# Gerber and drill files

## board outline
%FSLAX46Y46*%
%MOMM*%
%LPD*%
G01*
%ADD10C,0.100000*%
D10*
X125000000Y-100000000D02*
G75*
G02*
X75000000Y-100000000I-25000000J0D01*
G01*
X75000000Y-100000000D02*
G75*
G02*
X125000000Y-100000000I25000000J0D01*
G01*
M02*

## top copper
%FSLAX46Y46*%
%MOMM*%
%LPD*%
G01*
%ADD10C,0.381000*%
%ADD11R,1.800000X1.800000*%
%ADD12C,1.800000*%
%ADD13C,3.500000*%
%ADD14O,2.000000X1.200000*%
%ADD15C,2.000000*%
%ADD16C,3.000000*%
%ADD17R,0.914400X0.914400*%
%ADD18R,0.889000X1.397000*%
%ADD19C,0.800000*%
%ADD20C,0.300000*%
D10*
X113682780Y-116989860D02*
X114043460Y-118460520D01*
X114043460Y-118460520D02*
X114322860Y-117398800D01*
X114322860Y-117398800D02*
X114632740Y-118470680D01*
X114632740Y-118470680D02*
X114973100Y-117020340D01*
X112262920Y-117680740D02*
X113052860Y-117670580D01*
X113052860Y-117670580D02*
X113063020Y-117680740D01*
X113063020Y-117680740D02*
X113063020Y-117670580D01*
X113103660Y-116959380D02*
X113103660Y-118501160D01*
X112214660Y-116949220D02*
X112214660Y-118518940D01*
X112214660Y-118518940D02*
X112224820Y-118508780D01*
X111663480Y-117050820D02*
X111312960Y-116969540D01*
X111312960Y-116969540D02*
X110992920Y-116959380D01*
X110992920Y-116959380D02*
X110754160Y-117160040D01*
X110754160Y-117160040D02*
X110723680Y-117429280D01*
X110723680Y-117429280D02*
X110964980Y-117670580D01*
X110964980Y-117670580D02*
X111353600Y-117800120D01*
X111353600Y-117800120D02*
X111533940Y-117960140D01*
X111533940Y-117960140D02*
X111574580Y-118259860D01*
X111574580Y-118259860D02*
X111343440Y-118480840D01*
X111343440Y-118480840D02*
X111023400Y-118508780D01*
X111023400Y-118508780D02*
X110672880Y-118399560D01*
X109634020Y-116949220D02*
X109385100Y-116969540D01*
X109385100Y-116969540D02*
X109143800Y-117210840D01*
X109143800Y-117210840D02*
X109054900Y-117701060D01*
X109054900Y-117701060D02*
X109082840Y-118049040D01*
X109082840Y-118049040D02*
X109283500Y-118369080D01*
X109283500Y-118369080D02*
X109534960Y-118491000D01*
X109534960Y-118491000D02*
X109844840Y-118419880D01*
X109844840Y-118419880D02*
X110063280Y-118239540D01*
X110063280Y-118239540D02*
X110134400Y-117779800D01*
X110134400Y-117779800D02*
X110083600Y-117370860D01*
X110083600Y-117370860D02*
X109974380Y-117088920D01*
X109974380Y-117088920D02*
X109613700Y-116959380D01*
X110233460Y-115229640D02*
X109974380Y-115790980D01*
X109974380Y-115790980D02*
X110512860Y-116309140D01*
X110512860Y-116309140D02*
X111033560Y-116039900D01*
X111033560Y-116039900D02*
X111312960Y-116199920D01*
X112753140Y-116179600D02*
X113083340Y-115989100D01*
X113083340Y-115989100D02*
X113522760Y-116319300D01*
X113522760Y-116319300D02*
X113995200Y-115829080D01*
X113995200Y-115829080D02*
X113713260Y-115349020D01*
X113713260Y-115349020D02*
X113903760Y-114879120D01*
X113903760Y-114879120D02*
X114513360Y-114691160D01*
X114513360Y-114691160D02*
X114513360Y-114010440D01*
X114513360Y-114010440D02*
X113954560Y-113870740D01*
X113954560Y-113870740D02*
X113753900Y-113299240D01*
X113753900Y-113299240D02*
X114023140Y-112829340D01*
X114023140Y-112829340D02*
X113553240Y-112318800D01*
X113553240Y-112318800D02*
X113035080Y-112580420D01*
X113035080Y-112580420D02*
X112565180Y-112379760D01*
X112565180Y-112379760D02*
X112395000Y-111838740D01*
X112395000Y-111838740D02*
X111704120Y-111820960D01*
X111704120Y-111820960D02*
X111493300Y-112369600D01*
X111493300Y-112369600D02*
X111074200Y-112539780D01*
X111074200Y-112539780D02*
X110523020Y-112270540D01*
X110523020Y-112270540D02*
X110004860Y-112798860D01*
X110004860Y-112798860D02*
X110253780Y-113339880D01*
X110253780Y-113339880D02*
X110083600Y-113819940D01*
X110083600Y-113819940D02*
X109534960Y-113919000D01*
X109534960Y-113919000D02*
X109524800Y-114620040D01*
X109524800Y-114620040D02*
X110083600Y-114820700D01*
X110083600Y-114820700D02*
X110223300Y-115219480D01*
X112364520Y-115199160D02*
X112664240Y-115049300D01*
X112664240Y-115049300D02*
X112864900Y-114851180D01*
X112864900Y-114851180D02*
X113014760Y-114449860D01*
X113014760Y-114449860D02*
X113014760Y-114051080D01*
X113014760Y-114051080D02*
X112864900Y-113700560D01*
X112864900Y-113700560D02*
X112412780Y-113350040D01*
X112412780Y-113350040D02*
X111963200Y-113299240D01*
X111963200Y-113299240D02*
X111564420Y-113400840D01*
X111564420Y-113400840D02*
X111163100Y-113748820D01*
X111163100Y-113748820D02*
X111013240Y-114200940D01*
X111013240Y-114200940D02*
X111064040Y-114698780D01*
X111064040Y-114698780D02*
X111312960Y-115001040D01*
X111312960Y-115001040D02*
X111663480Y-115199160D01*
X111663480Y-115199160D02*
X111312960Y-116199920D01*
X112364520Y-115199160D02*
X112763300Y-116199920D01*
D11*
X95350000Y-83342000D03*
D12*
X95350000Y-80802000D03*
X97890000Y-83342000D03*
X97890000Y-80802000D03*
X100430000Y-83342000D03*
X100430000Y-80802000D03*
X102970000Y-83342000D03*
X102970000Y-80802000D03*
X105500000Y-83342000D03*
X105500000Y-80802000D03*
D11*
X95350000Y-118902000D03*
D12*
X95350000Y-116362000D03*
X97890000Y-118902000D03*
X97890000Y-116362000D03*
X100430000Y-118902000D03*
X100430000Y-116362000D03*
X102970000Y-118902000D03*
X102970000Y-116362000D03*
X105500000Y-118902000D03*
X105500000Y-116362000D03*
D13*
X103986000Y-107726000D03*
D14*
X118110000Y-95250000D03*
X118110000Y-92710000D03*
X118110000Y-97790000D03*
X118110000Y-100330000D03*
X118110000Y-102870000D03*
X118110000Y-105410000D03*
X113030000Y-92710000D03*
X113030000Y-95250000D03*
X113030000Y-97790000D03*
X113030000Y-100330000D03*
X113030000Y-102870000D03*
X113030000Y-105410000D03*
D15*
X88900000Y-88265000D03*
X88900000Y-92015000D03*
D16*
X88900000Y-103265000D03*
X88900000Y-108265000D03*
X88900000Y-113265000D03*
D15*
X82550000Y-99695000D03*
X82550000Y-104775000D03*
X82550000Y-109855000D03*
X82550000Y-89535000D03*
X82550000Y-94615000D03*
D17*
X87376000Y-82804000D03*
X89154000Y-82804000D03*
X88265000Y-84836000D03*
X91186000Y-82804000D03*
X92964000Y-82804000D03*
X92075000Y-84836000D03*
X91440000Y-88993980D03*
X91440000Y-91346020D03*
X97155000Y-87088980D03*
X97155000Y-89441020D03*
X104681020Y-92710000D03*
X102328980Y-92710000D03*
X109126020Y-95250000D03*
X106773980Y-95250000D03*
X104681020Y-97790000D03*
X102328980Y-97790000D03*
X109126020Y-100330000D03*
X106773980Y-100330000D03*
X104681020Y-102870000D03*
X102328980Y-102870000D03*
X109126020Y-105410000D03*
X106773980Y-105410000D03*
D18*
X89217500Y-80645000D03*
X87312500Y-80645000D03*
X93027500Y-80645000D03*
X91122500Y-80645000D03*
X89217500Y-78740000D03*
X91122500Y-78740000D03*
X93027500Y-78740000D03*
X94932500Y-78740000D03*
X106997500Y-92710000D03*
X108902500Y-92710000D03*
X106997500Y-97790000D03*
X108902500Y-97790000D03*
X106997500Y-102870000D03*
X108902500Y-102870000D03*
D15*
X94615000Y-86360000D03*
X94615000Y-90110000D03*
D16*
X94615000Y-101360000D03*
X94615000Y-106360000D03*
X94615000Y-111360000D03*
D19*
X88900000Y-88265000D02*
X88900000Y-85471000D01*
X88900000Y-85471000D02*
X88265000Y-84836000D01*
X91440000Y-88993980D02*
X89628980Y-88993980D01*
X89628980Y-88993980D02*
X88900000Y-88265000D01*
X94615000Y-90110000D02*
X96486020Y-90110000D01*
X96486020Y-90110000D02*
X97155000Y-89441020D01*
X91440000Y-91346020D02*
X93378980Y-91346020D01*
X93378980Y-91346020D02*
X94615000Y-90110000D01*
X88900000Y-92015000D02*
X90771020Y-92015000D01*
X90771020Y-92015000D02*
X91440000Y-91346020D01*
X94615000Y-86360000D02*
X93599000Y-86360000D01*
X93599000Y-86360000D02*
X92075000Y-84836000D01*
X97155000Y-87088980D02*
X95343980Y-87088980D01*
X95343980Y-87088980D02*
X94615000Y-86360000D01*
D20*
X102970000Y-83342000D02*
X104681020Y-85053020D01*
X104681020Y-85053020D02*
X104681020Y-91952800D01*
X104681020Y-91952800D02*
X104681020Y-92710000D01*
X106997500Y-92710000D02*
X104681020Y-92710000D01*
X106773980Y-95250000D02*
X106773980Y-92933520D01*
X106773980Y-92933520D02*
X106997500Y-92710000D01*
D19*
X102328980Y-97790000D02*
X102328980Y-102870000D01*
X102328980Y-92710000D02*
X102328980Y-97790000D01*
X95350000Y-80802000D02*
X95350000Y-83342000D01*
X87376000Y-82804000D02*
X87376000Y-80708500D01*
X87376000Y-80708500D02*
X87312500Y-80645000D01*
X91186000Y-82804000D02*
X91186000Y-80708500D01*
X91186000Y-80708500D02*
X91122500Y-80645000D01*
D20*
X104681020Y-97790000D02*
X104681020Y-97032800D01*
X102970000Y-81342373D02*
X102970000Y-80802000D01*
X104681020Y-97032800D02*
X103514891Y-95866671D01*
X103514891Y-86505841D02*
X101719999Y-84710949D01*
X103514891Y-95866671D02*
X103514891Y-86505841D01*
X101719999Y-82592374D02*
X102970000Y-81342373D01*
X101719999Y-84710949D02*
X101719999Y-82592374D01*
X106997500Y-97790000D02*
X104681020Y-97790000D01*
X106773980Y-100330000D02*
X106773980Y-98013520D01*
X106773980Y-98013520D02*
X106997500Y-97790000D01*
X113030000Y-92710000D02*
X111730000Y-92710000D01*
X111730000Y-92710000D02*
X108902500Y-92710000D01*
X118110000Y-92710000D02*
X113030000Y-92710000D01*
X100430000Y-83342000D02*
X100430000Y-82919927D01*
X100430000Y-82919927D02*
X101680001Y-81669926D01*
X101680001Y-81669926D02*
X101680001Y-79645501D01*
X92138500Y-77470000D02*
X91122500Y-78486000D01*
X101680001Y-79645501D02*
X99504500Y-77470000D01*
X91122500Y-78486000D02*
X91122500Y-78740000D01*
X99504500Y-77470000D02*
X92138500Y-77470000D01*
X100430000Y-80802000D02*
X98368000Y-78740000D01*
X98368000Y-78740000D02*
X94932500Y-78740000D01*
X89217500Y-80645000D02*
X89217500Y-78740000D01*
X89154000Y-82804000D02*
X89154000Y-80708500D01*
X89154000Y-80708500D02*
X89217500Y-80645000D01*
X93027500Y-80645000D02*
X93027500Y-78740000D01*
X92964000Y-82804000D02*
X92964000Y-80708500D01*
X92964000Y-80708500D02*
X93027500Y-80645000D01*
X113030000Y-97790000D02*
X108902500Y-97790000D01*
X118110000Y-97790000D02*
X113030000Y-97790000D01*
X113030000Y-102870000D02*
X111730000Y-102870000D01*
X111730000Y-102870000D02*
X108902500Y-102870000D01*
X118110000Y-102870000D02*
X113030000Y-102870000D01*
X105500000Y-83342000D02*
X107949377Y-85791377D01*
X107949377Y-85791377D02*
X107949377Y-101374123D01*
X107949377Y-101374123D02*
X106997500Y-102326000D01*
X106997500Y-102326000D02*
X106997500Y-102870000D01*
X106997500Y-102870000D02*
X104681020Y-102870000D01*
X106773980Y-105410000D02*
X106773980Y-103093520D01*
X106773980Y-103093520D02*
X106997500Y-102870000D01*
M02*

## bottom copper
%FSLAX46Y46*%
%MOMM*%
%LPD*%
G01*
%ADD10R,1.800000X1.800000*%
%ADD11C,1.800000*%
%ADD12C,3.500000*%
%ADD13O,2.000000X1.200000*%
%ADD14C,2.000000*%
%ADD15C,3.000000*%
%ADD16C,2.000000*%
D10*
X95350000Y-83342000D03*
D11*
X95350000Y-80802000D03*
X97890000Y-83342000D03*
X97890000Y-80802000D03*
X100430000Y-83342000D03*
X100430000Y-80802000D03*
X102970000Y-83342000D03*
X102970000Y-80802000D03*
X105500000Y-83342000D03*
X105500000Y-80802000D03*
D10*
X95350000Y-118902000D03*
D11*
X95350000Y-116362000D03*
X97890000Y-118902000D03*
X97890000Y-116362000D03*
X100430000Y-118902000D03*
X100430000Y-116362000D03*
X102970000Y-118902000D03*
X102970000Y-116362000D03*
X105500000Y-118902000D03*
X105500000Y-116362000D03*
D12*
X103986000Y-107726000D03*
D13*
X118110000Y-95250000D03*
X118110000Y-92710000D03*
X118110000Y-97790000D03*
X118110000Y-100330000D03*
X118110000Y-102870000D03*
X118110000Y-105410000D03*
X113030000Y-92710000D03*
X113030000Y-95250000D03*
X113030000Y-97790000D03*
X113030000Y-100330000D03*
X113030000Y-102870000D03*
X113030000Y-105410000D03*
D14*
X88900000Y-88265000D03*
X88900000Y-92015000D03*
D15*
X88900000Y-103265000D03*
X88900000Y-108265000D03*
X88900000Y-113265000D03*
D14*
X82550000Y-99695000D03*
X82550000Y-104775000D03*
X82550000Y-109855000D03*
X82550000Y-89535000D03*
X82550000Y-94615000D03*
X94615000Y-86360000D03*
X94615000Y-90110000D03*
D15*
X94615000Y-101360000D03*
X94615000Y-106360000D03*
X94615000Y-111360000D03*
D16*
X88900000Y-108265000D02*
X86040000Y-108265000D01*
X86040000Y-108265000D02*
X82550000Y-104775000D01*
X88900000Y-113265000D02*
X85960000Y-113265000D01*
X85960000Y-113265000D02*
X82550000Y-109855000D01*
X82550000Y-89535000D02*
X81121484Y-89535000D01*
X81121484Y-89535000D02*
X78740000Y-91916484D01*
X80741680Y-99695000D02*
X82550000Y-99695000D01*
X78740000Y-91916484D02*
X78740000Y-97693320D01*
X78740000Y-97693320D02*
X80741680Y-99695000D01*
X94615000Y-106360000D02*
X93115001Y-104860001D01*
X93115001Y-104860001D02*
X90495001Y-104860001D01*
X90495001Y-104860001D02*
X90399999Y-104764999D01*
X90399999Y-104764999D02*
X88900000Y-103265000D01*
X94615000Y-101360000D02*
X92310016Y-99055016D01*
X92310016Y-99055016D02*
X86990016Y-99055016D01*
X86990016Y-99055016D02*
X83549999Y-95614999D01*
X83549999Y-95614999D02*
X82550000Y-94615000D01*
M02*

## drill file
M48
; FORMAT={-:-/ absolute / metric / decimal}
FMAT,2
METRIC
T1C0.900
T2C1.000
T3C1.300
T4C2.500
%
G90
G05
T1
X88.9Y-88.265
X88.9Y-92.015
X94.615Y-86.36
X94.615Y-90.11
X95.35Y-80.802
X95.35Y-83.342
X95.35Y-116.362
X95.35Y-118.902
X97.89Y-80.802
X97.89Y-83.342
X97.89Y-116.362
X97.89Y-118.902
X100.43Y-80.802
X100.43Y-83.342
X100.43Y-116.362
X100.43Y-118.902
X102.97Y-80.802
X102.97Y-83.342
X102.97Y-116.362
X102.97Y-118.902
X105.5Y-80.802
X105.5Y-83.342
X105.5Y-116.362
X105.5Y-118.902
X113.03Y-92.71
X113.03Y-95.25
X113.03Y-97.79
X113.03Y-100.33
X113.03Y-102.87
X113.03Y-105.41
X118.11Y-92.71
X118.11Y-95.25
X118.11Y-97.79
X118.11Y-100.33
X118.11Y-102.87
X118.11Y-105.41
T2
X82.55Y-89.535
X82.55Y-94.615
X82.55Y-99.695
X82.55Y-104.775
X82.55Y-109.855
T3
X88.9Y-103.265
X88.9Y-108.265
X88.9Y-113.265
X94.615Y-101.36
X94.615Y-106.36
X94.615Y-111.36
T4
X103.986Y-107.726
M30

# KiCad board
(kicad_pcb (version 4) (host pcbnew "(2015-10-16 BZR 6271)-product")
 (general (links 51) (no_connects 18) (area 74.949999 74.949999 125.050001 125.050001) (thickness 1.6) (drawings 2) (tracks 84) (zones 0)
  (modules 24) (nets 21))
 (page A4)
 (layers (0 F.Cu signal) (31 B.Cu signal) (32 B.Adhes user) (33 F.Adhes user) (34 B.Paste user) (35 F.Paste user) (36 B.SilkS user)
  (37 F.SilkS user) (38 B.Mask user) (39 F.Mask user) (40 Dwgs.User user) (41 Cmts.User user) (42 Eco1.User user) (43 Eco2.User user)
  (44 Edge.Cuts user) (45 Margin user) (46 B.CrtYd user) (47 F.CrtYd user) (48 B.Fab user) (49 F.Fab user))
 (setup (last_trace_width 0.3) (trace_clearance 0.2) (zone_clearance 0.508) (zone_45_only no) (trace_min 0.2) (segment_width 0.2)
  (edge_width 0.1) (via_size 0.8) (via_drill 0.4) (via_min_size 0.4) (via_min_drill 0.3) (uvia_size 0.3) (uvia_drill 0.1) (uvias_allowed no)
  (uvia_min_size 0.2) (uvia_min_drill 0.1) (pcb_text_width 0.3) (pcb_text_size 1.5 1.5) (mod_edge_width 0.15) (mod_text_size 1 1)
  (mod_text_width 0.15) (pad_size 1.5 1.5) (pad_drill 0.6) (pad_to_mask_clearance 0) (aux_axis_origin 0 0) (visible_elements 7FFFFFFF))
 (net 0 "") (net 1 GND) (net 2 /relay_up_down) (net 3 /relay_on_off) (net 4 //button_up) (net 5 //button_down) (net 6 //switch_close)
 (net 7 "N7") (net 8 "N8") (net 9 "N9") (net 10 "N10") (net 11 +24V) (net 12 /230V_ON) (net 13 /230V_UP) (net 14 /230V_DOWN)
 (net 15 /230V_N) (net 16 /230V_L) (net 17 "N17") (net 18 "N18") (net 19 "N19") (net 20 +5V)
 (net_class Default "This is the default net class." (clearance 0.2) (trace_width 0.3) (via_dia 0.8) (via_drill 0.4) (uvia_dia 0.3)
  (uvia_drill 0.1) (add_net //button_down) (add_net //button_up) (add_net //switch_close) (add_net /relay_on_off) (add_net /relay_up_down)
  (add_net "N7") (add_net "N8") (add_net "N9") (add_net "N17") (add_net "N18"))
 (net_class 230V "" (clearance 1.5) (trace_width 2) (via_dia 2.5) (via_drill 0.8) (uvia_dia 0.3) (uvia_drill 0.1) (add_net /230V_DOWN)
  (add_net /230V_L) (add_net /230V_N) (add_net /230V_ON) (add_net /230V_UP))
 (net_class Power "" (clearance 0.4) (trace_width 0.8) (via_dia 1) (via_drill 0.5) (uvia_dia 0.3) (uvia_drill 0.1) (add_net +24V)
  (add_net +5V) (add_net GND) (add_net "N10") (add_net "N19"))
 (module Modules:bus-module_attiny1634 (layer B.Cu) (at 95.504 83.312 180)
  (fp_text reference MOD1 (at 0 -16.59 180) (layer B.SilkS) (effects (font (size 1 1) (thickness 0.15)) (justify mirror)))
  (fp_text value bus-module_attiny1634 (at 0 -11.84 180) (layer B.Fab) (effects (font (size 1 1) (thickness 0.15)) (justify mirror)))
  (pad 1 thru_hole rect (at 0.154 -0.03 180) (size 1.8 1.8) (drill 0.9) (layers *.Cu *.Mask B.SilkS) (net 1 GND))
  (pad 2 thru_hole circle (at 0.154 2.51 180) (size 1.8 1.8) (drill 0.9) (layers *.Cu *.Mask B.SilkS) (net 1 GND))
  (pad 3 thru_hole circle (at -2.386 -0.03 180) (size 1.8 1.8) (drill 0.9) (layers *.Cu *.Mask B.SilkS))
  (pad 4 thru_hole circle (at -2.386 2.51 180) (size 1.8 1.8) (drill 0.9) (layers *.Cu *.Mask B.SilkS))
  (pad 5 thru_hole circle (at -4.926 -0.03 180) (size 1.8 1.8) (drill 0.9) (layers *.Cu *.Mask B.SilkS) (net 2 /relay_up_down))
  (pad 6 thru_hole circle (at -4.926 2.51 180) (size 1.8 1.8) (drill 0.9) (layers *.Cu *.Mask B.SilkS) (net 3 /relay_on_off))
  (pad 7 thru_hole circle (at -7.466 -0.03 180) (size 1.8 1.8) (drill 0.9) (layers *.Cu *.Mask B.SilkS) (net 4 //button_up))
  (pad 8 thru_hole circle (at -7.466 2.51 180) (size 1.8 1.8) (drill 0.9) (layers *.Cu *.Mask B.SilkS) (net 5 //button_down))
  (pad 9 thru_hole circle (at -9.996 -0.03 180) (size 1.8 1.8) (drill 0.9) (layers *.Cu *.Mask B.SilkS) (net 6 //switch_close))
  (pad 10 thru_hole circle (at -9.996 2.51 180) (size 1.8 1.8) (drill 0.9) (layers *.Cu *.Mask B.SilkS))
  (pad 11 thru_hole rect (at 0.154 -35.59 180) (size 1.8 1.8) (drill 0.9) (layers *.Cu *.Mask B.SilkS) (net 1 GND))
  (pad 12 thru_hole circle (at 0.154 -33.05 180) (size 1.8 1.8) (drill 0.9) (layers *.Cu *.Mask B.SilkS) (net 1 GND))
  (pad 13 thru_hole circle (at -2.386 -35.59 180) (size 1.8 1.8) (drill 0.9) (layers *.Cu *.Mask B.SilkS))
  (pad 14 thru_hole circle (at -2.386 -33.05 180) (size 1.8 1.8) (drill 0.9) (layers *.Cu *.Mask B.SilkS))
  (pad 15 thru_hole circle (at -4.926 -35.59 180) (size 1.8 1.8) (drill 0.9) (layers *.Cu *.Mask B.SilkS))
  (pad 16 thru_hole circle (at -4.926 -33.05 180) (size 1.8 1.8) (drill 0.9) (layers *.Cu *.Mask B.SilkS))
  (pad 17 thru_hole circle (at -7.466 -35.59 180) (size 1.8 1.8) (drill 0.9) (layers *.Cu *.Mask B.SilkS))
  (pad 18 thru_hole circle (at -7.466 -33.05 180) (size 1.8 1.8) (drill 0.9) (layers *.Cu *.Mask B.SilkS))
  (pad 19 thru_hole circle (at -9.996 -35.59 180) (size 1.8 1.8) (drill 0.9) (layers *.Cu *.Mask B.SilkS))
  (pad 20 thru_hole circle (at -9.996 -33.05 180) (size 1.8 1.8) (drill 0.9) (layers *.Cu *.Mask B.SilkS))
  (pad 21 thru_hole circle (at -8.482 -24.414 180) (size 3.5 3.5) (drill 2.5) (layers *.Cu *.Mask B.SilkS)))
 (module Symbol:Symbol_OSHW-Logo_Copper (layer F.Cu) (at 112.014 114.3)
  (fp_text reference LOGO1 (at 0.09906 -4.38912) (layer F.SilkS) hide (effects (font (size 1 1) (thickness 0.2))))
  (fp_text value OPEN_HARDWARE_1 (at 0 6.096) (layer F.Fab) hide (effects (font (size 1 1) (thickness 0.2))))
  (fp_line (start 1.66878 2.68986) (end 2.02946 4.16052) (layer F.Cu) (width 0.381))
  (fp_line (start 2.02946 4.16052) (end 2.30886 3.0988) (layer F.Cu) (width 0.381))
  (fp_line (start 2.30886 3.0988) (end 2.61874 4.17068) (layer F.Cu) (width 0.381))
  (fp_line (start 2.61874 4.17068) (end 2.9591 2.72034) (layer F.Cu) (width 0.381))
  (fp_line (start 0.24892 3.38074) (end 1.03886 3.37058) (layer F.Cu) (width 0.381))
  (fp_line (start 1.03886 3.37058) (end 1.04902 3.38074) (layer F.Cu) (width 0.381))
  (fp_line (start 1.04902 3.38074) (end 1.04902 3.37058) (layer F.Cu) (width 0.381))
  (fp_line (start 1.08966 2.65938) (end 1.08966 4.20116) (layer F.Cu) (width 0.381))
  (fp_line (start 0.20066 2.64922) (end 0.20066 4.21894) (layer F.Cu) (width 0.381))
  (fp_line (start 0.20066 4.21894) (end 0.21082 4.20878) (layer F.Cu) (width 0.381))
  (fp_line (start -0.35052 2.75082) (end -0.70104 2.66954) (layer F.Cu) (width 0.381))
  (fp_line (start -0.70104 2.66954) (end -1.02108 2.65938) (layer F.Cu) (width 0.381))
  (fp_line (start -1.02108 2.65938) (end -1.25984 2.86004) (layer F.Cu) (width 0.381))
  (fp_line (start -1.25984 2.86004) (end -1.29032 3.12928) (layer F.Cu) (width 0.381))
  (fp_line (start -1.29032 3.12928) (end -1.04902 3.37058) (layer F.Cu) (width 0.381))
  (fp_line (start -1.04902 3.37058) (end -0.6604 3.50012) (layer F.Cu) (width 0.381))
  (fp_line (start -0.6604 3.50012) (end -0.48006 3.66014) (layer F.Cu) (width 0.381))
  (fp_line (start -0.48006 3.66014) (end -0.43942 3.95986) (layer F.Cu) (width 0.381))
  (fp_line (start -0.43942 3.95986) (end -0.67056 4.18084) (layer F.Cu) (width 0.381))
  (fp_line (start -0.67056 4.18084) (end -0.9906 4.20878) (layer F.Cu) (width 0.381))
  (fp_line (start -0.9906 4.20878) (end -1.34112 4.09956) (layer F.Cu) (width 0.381))
  (fp_line (start -2.37998 2.64922) (end -2.6289 2.66954) (layer F.Cu) (width 0.381))
  (fp_line (start -2.6289 2.66954) (end -2.8702 2.91084) (layer F.Cu) (width 0.381))
  (fp_line (start -2.8702 2.91084) (end -2.9591 3.40106) (layer F.Cu) (width 0.381))
  (fp_line (start -2.9591 3.40106) (end -2.93116 3.74904) (layer F.Cu) (width 0.381))
  (fp_line (start -2.93116 3.74904) (end -2.7305 4.06908) (layer F.Cu) (width 0.381))
  (fp_line (start -2.7305 4.06908) (end -2.47904 4.191) (layer F.Cu) (width 0.381))
  (fp_line (start -2.47904 4.191) (end -2.16916 4.11988) (layer F.Cu) (width 0.381))
  (fp_line (start -2.16916 4.11988) (end -1.95072 3.93954) (layer F.Cu) (width 0.381))
  (fp_line (start -1.95072 3.93954) (end -1.8796 3.4798) (layer F.Cu) (width 0.381))
  (fp_line (start -1.8796 3.4798) (end -1.9304 3.07086) (layer F.Cu) (width 0.381))
  (fp_line (start -1.9304 3.07086) (end -2.03962 2.78892) (layer F.Cu) (width 0.381))
  (fp_line (start -2.03962 2.78892) (end -2.4003 2.65938) (layer F.Cu) (width 0.381))
  (fp_line (start -1.78054 0.92964) (end -2.03962 1.49098) (layer F.Cu) (width 0.381))
  (fp_line (start -2.03962 1.49098) (end -1.50114 2.00914) (layer F.Cu) (width 0.381))
  (fp_line (start -1.50114 2.00914) (end -0.98044 1.7399) (layer F.Cu) (width 0.381))
  (fp_line (start -0.98044 1.7399) (end -0.70104 1.89992) (layer F.Cu) (width 0.381))
  (fp_line (start 0.73914 1.8796) (end 1.06934 1.6891) (layer F.Cu) (width 0.381))
  (fp_line (start 1.06934 1.6891) (end 1.50876 2.0193) (layer F.Cu) (width 0.381))
  (fp_line (start 1.50876 2.0193) (end 1.9812 1.52908) (layer F.Cu) (width 0.381))
  (fp_line (start 1.9812 1.52908) (end 1.69926 1.04902) (layer F.Cu) (width 0.381))
  (fp_line (start 1.69926 1.04902) (end 1.88976 0.57912) (layer F.Cu) (width 0.381))
  (fp_line (start 1.88976 0.57912) (end 2.49936 0.39116) (layer F.Cu) (width 0.381))
  (fp_line (start 2.49936 0.39116) (end 2.49936 -0.28956) (layer F.Cu) (width 0.381))
  (fp_line (start 2.49936 -0.28956) (end 1.94056 -0.42926) (layer F.Cu) (width 0.381))
  (fp_line (start 1.94056 -0.42926) (end 1.7399 -1.00076) (layer F.Cu) (width 0.381))
  (fp_line (start 1.7399 -1.00076) (end 2.00914 -1.47066) (layer F.Cu) (width 0.381))
  (fp_line (start 2.00914 -1.47066) (end 1.53924 -1.9812) (layer F.Cu) (width 0.381))
  (fp_line (start 1.53924 -1.9812) (end 1.02108 -1.71958) (layer F.Cu) (width 0.381))
  (fp_line (start 1.02108 -1.71958) (end 0.55118 -1.92024) (layer F.Cu) (width 0.381))
  (fp_line (start 0.55118 -1.92024) (end 0.381 -2.46126) (layer F.Cu) (width 0.381))
  (fp_line (start 0.381 -2.46126) (end -0.30988 -2.47904) (layer F.Cu) (width 0.381))
  (fp_line (start -0.30988 -2.47904) (end -0.5207 -1.9304) (layer F.Cu) (width 0.381))
  (fp_line (start -0.5207 -1.9304) (end -0.9398 -1.76022) (layer F.Cu) (width 0.381))
  (fp_line (start -0.9398 -1.76022) (end -1.49098 -2.02946) (layer F.Cu) (width 0.381))
  (fp_line (start -1.49098 -2.02946) (end -2.00914 -1.50114) (layer F.Cu) (width 0.381))
  (fp_line (start -2.00914 -1.50114) (end -1.76022 -0.96012) (layer F.Cu) (width 0.381))
  (fp_line (start -1.76022 -0.96012) (end -1.9304 -0.48006) (layer F.Cu) (width 0.381))
  (fp_line (start -1.9304 -0.48006) (end -2.47904 -0.381) (layer F.Cu) (width 0.381))
  (fp_line (start -2.47904 -0.381) (end -2.4892 0.32004) (layer F.Cu) (width 0.381))
  (fp_line (start -2.4892 0.32004) (end -1.9304 0.5207) (layer F.Cu) (width 0.381))
  (fp_line (start -1.9304 0.5207) (end -1.7907 0.91948) (layer F.Cu) (width 0.381))
  (fp_line (start 0.35052 0.89916) (end 0.65024 0.7493) (layer F.Cu) (width 0.381))
  (fp_line (start 0.65024 0.7493) (end 0.8509 0.55118) (layer F.Cu) (width 0.381))
  (fp_line (start 0.8509 0.55118) (end 1.00076 0.14986) (layer F.Cu) (width 0.381))
  (fp_line (start 1.00076 0.14986) (end 1.00076 -0.24892) (layer F.Cu) (width 0.381))
  (fp_line (start 1.00076 -0.24892) (end 0.8509 -0.59944) (layer F.Cu) (width 0.381))
  (fp_line (start 0.8509 -0.59944) (end 0.39878 -0.94996) (layer F.Cu) (width 0.381))
  (fp_line (start 0.39878 -0.94996) (end -0.0508 -1.00076) (layer F.Cu) (width 0.381))
  (fp_line (start -0.0508 -1.00076) (end -0.44958 -0.89916) (layer F.Cu) (width 0.381))
  (fp_line (start -0.44958 -0.89916) (end -0.8509 -0.55118) (layer F.Cu) (width 0.381))
  (fp_line (start -0.8509 -0.55118) (end -1.00076 -0.09906) (layer F.Cu) (width 0.381))
  (fp_line (start -1.00076 -0.09906) (end -0.94996 0.39878) (layer F.Cu) (width 0.381))
  (fp_line (start -0.94996 0.39878) (end -0.70104 0.70104) (layer F.Cu) (width 0.381))
  (fp_line (start -0.70104 0.70104) (end -0.35052 0.89916) (layer F.Cu) (width 0.381))
  (fp_line (start -0.35052 0.89916) (end -0.70104 1.89992) (layer F.Cu) (width 0.381))
  (fp_line (start 0.35052 0.89916) (end 0.7493 1.89992) (layer F.Cu) (width 0.381)))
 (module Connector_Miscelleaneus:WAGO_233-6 (layer F.Cu) (at 118.11 92.71 270)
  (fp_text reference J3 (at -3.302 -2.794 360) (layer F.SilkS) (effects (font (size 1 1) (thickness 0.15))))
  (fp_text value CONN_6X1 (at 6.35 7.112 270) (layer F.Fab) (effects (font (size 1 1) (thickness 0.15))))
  (pad 2 thru_hole oval (at 2.54 0 270) (size 1.2 2) (drill 0.9) (layers *.Cu *.Mask F.SilkS) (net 1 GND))
  (pad 1 thru_hole oval (at 0 0 270) (size 1.2 2) (drill 0.9) (layers *.Cu *.Mask F.SilkS) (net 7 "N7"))
  (pad 3 thru_hole oval (at 5.08 0 270) (size 1.2 2) (drill 0.9) (layers *.Cu *.Mask F.SilkS) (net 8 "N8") (solder_mask_margin 0.1)
   (clearance 0.1))
  (pad 4 thru_hole oval (at 7.62 0 270) (size 1.2 2) (drill 0.9) (layers *.Cu *.Mask F.SilkS) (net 1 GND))
  (pad 5 thru_hole oval (at 10.16 0 270) (size 1.2 2) (drill 0.9) (layers *.Cu *.Mask F.SilkS) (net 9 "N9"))
  (pad 6 thru_hole oval (at 12.7 0 270) (size 1.2 2) (drill 0.9) (layers *.Cu *.Mask F.SilkS) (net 1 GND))
  (pad 1 thru_hole oval (at 0 5.08 270) (size 1.2 2) (drill 0.9) (layers *.Cu *.Mask F.SilkS) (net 7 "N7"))
  (pad 2 thru_hole oval (at 2.54 5.08 270) (size 1.2 2) (drill 0.9) (layers *.Cu *.Mask F.SilkS) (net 1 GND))
  (pad 3 thru_hole oval (at 5.08 5.08 270) (size 1.2 2) (drill 0.9) (layers *.Cu *.Mask F.SilkS) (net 8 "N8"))
  (pad 4 thru_hole oval (at 7.62 5.08 270) (size 1.2 2) (drill 0.9) (layers *.Cu *.Mask F.SilkS) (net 1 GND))
  (pad 5 thru_hole oval (at 10.16 5.08 270) (size 1.2 2) (drill 0.9) (layers *.Cu *.Mask F.SilkS) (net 9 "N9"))
  (pad 6 thru_hole oval (at 12.7 5.08 270) (size 1.2 2) (drill 0.9) (layers *.Cu *.Mask F.SilkS) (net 1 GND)))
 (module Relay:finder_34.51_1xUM (layer F.Cu) (at 88.9 88.265 270)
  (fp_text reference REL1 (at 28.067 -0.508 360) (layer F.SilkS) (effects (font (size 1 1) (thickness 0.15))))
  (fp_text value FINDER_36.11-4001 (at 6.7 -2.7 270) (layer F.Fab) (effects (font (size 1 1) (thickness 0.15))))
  (pad 1 thru_hole circle (at 0 0 270) (size 2 2) (drill 0.9) (layers *.Cu *.Mask F.SilkS) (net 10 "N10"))
  (pad 2 thru_hole circle (at 3.75 0 270) (size 2 2) (drill 0.9) (layers *.Cu *.Mask F.SilkS) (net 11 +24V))
  (pad 3 thru_hole circle (at 15 0 270) (size 3 3) (drill 1.3) (layers *.Cu *.Mask F.SilkS) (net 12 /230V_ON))
  (pad 4 thru_hole circle (at 20 0 270) (size 3 3) (drill 1.3) (layers *.Cu *.Mask F.SilkS) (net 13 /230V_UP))
  (pad 5 thru_hole circle (at 25 0 270) (size 3 3) (drill 1.3) (layers *.Cu *.Mask F.SilkS) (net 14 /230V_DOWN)))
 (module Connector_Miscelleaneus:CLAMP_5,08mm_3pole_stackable (layer F.Cu) (at 82.55 99.695 270)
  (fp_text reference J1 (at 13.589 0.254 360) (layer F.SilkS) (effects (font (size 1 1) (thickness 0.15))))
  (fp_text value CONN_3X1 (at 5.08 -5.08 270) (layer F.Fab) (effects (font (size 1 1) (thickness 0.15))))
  (pad 1 thru_hole circle (at 0 0 270) (size 2 2) (drill 1) (layers *.Cu *.Mask F.SilkS) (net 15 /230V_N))
  (pad 2 thru_hole circle (at 5.08 0 270) (size 2 2) (drill 1) (layers *.Cu *.Mask F.SilkS) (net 13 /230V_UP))
  (pad 3 thru_hole circle (at 10.16 0 270) (size 2 2) (drill 1) (layers *.Cu *.Mask F.SilkS) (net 14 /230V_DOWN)))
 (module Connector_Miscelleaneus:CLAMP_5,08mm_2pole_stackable (layer F.Cu) (at 82.55 89.535 270)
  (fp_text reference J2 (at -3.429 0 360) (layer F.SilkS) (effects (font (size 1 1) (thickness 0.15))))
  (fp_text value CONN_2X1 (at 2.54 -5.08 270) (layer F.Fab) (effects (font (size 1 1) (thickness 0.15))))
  (pad 1 thru_hole circle (at 0 0 270) (size 2 2) (drill 1) (layers *.Cu *.Mask F.SilkS) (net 15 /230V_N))
  (pad 2 thru_hole circle (at 5.08 0 270) (size 2 2) (drill 1) (layers *.Cu *.Mask F.SilkS) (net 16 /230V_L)))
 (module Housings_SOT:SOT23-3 (layer F.Cu) (at 88.265 83.82)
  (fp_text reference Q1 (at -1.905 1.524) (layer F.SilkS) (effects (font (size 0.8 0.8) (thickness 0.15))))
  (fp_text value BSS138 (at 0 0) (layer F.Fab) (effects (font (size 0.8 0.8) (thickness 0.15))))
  (pad 2 smd rect (at -0.889 -1.016) (size 0.9144 0.9144) (layers F.Cu F.Paste F.Mask) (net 1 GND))
  (pad 1 smd rect (at 0.889 -1.016) (size 0.9144 0.9144) (layers F.Cu F.Paste F.Mask) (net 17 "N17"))
  (pad 3 smd rect (at 0 1.016) (size 0.9144 0.9144) (layers F.Cu F.Paste F.Mask) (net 10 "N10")))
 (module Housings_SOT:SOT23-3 (layer F.Cu) (at 92.075 83.82)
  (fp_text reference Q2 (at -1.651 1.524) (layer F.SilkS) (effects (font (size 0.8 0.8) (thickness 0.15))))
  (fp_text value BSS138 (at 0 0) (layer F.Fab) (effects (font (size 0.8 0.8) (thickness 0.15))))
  (pad 2 smd rect (at -0.889 -1.016) (size 0.9144 0.9144) (layers F.Cu F.Paste F.Mask) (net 1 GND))
  (pad 1 smd rect (at 0.889 -1.016) (size 0.9144 0.9144) (layers F.Cu F.Paste F.Mask) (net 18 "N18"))
  (pad 3 smd rect (at 0 1.016) (size 0.9144 0.9144) (layers F.Cu F.Paste F.Mask) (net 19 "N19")))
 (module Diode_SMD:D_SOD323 (layer F.Cu) (at 91.44 90.17 270)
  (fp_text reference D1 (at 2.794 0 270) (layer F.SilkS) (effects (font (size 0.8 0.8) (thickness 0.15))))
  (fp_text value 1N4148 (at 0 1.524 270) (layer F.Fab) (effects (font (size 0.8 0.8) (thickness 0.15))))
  (pad 1 smd rect (at -1.17602 0 270) (size 0.9144 0.9144) (layers F.Cu F.Paste F.Mask) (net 10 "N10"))
  (pad 2 smd rect (at 1.17602 0 270) (size 0.9144 0.9144) (layers F.Cu F.Paste F.Mask) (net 11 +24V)))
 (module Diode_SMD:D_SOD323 (layer F.Cu) (at 97.155 88.265 270)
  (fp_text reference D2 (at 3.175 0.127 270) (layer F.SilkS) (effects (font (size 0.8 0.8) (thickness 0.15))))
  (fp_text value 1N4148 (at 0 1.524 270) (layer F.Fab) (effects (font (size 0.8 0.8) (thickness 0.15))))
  (pad 1 smd rect (at -1.17602 0 270) (size 0.9144 0.9144) (layers F.Cu F.Paste F.Mask) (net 19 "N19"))
  (pad 2 smd rect (at 1.17602 0 270) (size 0.9144 0.9144) (layers F.Cu F.Paste F.Mask) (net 11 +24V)))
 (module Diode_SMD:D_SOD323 (layer F.Cu) (at 103.505 92.71 180)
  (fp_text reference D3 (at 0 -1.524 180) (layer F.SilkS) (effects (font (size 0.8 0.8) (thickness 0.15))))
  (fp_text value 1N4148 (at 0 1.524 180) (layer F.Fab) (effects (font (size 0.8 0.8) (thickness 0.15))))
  (pad 1 smd rect (at -1.17602 0 180) (size 0.9144 0.9144) (layers F.Cu F.Paste F.Mask) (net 4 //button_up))
  (pad 2 smd rect (at 1.17602 0 180) (size 0.9144 0.9144) (layers F.Cu F.Paste F.Mask) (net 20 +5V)))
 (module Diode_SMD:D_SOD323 (layer F.Cu) (at 107.95 95.25 180)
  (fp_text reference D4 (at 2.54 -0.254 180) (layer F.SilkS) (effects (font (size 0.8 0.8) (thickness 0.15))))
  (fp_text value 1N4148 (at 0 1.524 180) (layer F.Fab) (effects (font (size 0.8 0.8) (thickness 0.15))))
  (pad 1 smd rect (at -1.17602 0 180) (size 0.9144 0.9144) (layers F.Cu F.Paste F.Mask) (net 1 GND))
  (pad 2 smd rect (at 1.17602 0 180) (size 0.9144 0.9144) (layers F.Cu F.Paste F.Mask) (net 4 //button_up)))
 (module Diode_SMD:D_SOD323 (layer F.Cu) (at 103.505 97.79 180)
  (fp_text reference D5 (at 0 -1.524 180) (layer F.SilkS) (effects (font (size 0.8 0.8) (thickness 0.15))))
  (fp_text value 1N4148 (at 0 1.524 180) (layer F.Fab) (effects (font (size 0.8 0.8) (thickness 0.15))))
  (pad 1 smd rect (at -1.17602 0 180) (size 0.9144 0.9144) (layers F.Cu F.Paste F.Mask) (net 5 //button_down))
  (pad 2 smd rect (at 1.17602 0 180) (size 0.9144 0.9144) (layers F.Cu F.Paste F.Mask) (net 20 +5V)))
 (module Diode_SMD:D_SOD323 (layer F.Cu) (at 107.95 100.33 180)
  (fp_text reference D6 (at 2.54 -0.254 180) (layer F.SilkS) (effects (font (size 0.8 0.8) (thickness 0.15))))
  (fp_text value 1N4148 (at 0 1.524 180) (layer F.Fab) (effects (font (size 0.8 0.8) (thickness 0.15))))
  (pad 1 smd rect (at -1.17602 0 180) (size 0.9144 0.9144) (layers F.Cu F.Paste F.Mask) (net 1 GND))
  (pad 2 smd rect (at 1.17602 0 180) (size 0.9144 0.9144) (layers F.Cu F.Paste F.Mask) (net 5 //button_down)))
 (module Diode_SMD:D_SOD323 (layer F.Cu) (at 103.505 102.87 180)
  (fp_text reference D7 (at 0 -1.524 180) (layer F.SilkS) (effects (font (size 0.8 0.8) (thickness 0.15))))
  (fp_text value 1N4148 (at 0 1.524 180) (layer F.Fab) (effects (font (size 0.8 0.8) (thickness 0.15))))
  (pad 1 smd rect (at -1.17602 0 180) (size 0.9144 0.9144) (layers F.Cu F.Paste F.Mask) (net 6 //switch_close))
  (pad 2 smd rect (at 1.17602 0 180) (size 0.9144 0.9144) (layers F.Cu F.Paste F.Mask) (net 20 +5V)))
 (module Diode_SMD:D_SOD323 (layer F.Cu) (at 107.95 105.41 180)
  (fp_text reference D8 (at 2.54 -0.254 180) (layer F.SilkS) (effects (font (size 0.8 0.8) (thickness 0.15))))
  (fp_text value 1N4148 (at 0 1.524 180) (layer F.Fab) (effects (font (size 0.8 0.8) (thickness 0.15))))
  (pad 1 smd rect (at -1.17602 0 180) (size 0.9144 0.9144) (layers F.Cu F.Paste F.Mask) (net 1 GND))
  (pad 2 smd rect (at 1.17602 0 180) (size 0.9144 0.9144) (layers F.Cu F.Paste F.Mask) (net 6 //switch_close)))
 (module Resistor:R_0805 (layer F.Cu) (at 88.265 80.645 180)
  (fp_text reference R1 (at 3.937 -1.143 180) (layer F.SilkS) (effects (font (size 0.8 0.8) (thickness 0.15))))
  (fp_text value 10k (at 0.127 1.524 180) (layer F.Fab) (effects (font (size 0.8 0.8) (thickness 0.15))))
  (pad 1 smd rect (at -0.9525 0 180) (size 0.889 1.397) (layers F.Cu F.Paste F.Mask) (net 17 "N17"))
  (pad 2 smd rect (at 0.9525 0 180) (size 0.889 1.397) (layers F.Cu F.Paste F.Mask) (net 1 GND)))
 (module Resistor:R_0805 (layer F.Cu) (at 92.075 80.645 180)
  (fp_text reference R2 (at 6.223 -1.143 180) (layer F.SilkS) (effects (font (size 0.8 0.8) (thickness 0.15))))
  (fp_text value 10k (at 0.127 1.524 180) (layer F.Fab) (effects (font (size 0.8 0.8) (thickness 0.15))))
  (pad 1 smd rect (at -0.9525 0 180) (size 0.889 1.397) (layers F.Cu F.Paste F.Mask) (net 18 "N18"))
  (pad 2 smd rect (at 0.9525 0 180) (size 0.889 1.397) (layers F.Cu F.Paste F.Mask) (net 1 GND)))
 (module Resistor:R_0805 (layer F.Cu) (at 90.17 78.74)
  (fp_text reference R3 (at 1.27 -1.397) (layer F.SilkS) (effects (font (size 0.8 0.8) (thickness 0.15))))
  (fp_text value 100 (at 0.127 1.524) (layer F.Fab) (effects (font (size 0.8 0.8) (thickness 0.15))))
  (pad 1 smd rect (at -0.9525 0) (size 0.889 1.397) (layers F.Cu F.Paste F.Mask) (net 17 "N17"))
  (pad 2 smd rect (at 0.9525 0) (size 0.889 1.397) (layers F.Cu F.Paste F.Mask) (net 2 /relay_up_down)))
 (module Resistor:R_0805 (layer F.Cu) (at 93.98 78.74)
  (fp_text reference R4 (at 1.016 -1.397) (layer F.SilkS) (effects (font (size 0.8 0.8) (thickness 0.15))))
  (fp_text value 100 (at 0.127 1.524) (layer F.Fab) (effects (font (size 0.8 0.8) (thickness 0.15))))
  (pad 1 smd rect (at -0.9525 0) (size 0.889 1.397) (layers F.Cu F.Paste F.Mask) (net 18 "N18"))
  (pad 2 smd rect (at 0.9525 0) (size 0.889 1.397) (layers F.Cu F.Paste F.Mask) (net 3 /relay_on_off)))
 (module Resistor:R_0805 (layer F.Cu) (at 107.95 92.71)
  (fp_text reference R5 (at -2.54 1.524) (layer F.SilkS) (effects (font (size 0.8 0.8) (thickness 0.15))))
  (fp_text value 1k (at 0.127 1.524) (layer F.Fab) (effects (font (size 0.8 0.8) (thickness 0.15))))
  (pad 1 smd rect (at -0.9525 0) (size 0.889 1.397) (layers F.Cu F.Paste F.Mask) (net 4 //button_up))
  (pad 2 smd rect (at 0.9525 0) (size 0.889 1.397) (layers F.Cu F.Paste F.Mask) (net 7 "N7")))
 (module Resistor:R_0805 (layer F.Cu) (at 107.95 97.79)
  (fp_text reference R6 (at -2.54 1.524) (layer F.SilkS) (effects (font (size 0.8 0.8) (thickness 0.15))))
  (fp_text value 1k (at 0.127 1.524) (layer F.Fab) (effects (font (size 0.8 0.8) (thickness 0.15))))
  (pad 1 smd rect (at -0.9525 0) (size 0.889 1.397) (layers F.Cu F.Paste F.Mask) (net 5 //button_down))
  (pad 2 smd rect (at 0.9525 0) (size 0.889 1.397) (layers F.Cu F.Paste F.Mask) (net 8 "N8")))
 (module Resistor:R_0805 (layer F.Cu) (at 107.95 102.87)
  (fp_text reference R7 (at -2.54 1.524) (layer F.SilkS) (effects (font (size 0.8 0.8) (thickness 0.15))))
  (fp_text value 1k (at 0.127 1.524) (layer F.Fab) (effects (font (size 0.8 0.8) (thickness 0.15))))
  (pad 1 smd rect (at -0.9525 0) (size 0.889 1.397) (layers F.Cu F.Paste F.Mask) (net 6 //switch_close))
  (pad 2 smd rect (at 0.9525 0) (size 0.889 1.397) (layers F.Cu F.Paste F.Mask) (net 9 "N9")))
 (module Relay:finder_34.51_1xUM (layer F.Cu) (at 94.615 86.36 270)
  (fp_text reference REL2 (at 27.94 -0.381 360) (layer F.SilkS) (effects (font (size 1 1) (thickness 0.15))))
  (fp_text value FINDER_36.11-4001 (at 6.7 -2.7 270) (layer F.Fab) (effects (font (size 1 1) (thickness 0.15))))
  (pad 1 thru_hole circle (at 0 0 270) (size 2 2) (drill 0.9) (layers *.Cu *.Mask F.SilkS) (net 19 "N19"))
  (pad 2 thru_hole circle (at 3.75 0 270) (size 2 2) (drill 0.9) (layers *.Cu *.Mask F.SilkS) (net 11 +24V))
  (pad 3 thru_hole circle (at 15 0 270) (size 3 3) (drill 1.3) (layers *.Cu *.Mask F.SilkS) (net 16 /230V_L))
  (pad 4 thru_hole circle (at 20 0 270) (size 3 3) (drill 1.3) (layers *.Cu *.Mask F.SilkS) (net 12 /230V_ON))
  (pad 5 thru_hole circle (at 25 0 270) (size 3 3) (drill 1.3) (layers *.Cu *.Mask F.SilkS)))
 (gr_circle (center 100 100) (end 125 100) (layer Edge.Cuts) (width 0.1))
 (segment (start 88.9 88.265) (end 88.9 85.471) (width 0.8) (layer F.Cu) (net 10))
 (segment (start 88.9 85.471) (end 88.265 84.836) (width 0.8) (layer F.Cu) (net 10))
 (segment (start 91.44 88.99398) (end 89.62898 88.99398) (width 0.8) (layer F.Cu) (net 10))
 (segment (start 89.62898 88.99398) (end 88.9 88.265) (width 0.8) (layer F.Cu) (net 10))
 (segment (start 94.615 90.11) (end 96.48602 90.11) (width 0.8) (layer F.Cu) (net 11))
 (segment (start 96.48602 90.11) (end 97.155 89.44102) (width 0.8) (layer F.Cu) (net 11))
 (segment (start 91.44 91.34602) (end 93.37898 91.34602) (width 0.8) (layer F.Cu) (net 11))
 (segment (start 93.37898 91.34602) (end 94.615 90.11) (width 0.8) (layer F.Cu) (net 11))
 (segment (start 88.9 92.015) (end 90.77102 92.015) (width 0.8) (layer F.Cu) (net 11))
 (segment (start 90.77102 92.015) (end 91.44 91.34602) (width 0.8) (layer F.Cu) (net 11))
 (segment (start 94.615 86.36) (end 93.599 86.36) (width 0.8) (layer F.Cu) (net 19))
 (segment (start 93.599 86.36) (end 92.075 84.836) (width 0.8) (layer F.Cu) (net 19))
 (segment (start 97.155 87.08898) (end 95.34398 87.08898) (width 0.8) (layer F.Cu) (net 19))
 (segment (start 95.34398 87.08898) (end 94.615 86.36) (width 0.8) (layer F.Cu) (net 19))
 (segment (start 102.97 83.342) (end 104.68102 85.05302) (width 0.3) (layer F.Cu) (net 4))
 (segment (start 104.68102 85.05302) (end 104.68102 91.9528) (width 0.3) (layer F.Cu) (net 4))
 (segment (start 104.68102 91.9528) (end 104.68102 92.71) (width 0.3) (layer F.Cu) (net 4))
 (segment (start 106.9975 92.71) (end 104.68102 92.71) (width 0.3) (layer F.Cu) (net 4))
 (segment (start 106.77398 95.25) (end 106.77398 92.93352) (width 0.3) (layer F.Cu) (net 4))
 (segment (start 106.77398 92.93352) (end 106.9975 92.71) (width 0.3) (layer F.Cu) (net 4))
 (segment (start 102.32898 97.79) (end 102.32898 102.87) (width 0.8) (layer F.Cu) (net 20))
 (segment (start 102.32898 92.71) (end 102.32898 97.79) (width 0.8) (layer F.Cu) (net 20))
 (segment (start 95.35 80.802) (end 95.35 83.342) (width 0.8) (layer F.Cu) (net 1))
 (segment (start 87.376 82.804) (end 87.376 80.7085) (width 0.8) (layer F.Cu) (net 1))
 (segment (start 87.376 80.7085) (end 87.3125 80.645) (width 0.8) (layer F.Cu) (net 1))
 (segment (start 91.186 82.804) (end 91.186 80.7085) (width 0.8) (layer F.Cu) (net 1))
 (segment (start 91.186 80.7085) (end 91.1225 80.645) (width 0.8) (layer F.Cu) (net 1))
 (segment (start 104.68102 97.79) (end 104.68102 97.0328) (width 0.3) (layer F.Cu) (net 5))
 (segment (start 102.97 81.342373) (end 102.97 80.802) (width 0.3) (layer F.Cu) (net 5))
 (segment (start 104.68102 97.0328) (end 103.514891 95.866671) (width 0.3) (layer F.Cu) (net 5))
 (segment (start 103.514891 86.505841) (end 101.719999 84.710949) (width 0.3) (layer F.Cu) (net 5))
 (segment (start 103.514891 95.866671) (end 103.514891 86.505841) (width 0.3) (layer F.Cu) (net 5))
 (segment (start 101.719999 82.592374) (end 102.97 81.342373) (width 0.3) (layer F.Cu) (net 5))
 (segment (start 101.719999 84.710949) (end 101.719999 82.592374) (width 0.3) (layer F.Cu) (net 5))
 (segment (start 106.9975 97.79) (end 104.68102 97.79) (width 0.3) (layer F.Cu) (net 5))
 (segment (start 106.77398 100.33) (end 106.77398 98.01352) (width 0.3) (layer F.Cu) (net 5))
 (segment (start 106.77398 98.01352) (end 106.9975 97.79) (width 0.3) (layer F.Cu) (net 5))
 (segment (start 113.03 92.71) (end 111.73 92.71) (width 0.3) (layer F.Cu) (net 7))
 (segment (start 111.73 92.71) (end 108.9025 92.71) (width 0.3) (layer F.Cu) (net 7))
 (segment (start 118.11 92.71) (end 113.03 92.71) (width 0.3) (layer F.Cu) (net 7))
 (segment (start 100.43 83.342) (end 100.43 82.919927) (width 0.3) (layer F.Cu) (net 2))
 (segment (start 100.43 82.919927) (end 101.680001 81.669926) (width 0.3) (layer F.Cu) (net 2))
 (segment (start 101.680001 81.669926) (end 101.680001 79.645501) (width 0.3) (layer F.Cu) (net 2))
 (segment (start 92.1385 77.47) (end 91.1225 78.486) (width 0.3) (layer F.Cu) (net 2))
 (segment (start 101.680001 79.645501) (end 99.5045 77.47) (width 0.3) (layer F.Cu) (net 2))
 (segment (start 91.1225 78.486) (end 91.1225 78.74) (width 0.3) (layer F.Cu) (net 2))
 (segment (start 99.5045 77.47) (end 92.1385 77.47) (width 0.3) (layer F.Cu) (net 2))
 (segment (start 100.43 80.802) (end 98.368 78.74) (width 0.3) (layer F.Cu) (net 3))
 (segment (start 98.368 78.74) (end 94.9325 78.74) (width 0.3) (layer F.Cu) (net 3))
 (segment (start 89.2175 80.645) (end 89.2175 78.74) (width 0.3) (layer F.Cu) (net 17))
 (segment (start 89.154 82.804) (end 89.154 80.7085) (width 0.3) (layer F.Cu) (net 17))
 (segment (start 89.154 80.7085) (end 89.2175 80.645) (width 0.3) (layer F.Cu) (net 17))
 (segment (start 93.0275 80.645) (end 93.0275 78.74) (width 0.3) (layer F.Cu) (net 18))
 (segment (start 92.964 82.804) (end 92.964 80.7085) (width 0.3) (layer F.Cu) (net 18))
 (segment (start 92.964 80.7085) (end 93.0275 80.645) (width 0.3) (layer F.Cu) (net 18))
 (segment (start 113.03 97.79) (end 108.9025 97.79) (width 0.3) (layer F.Cu) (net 8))
 (segment (start 118.11 97.79) (end 113.03 97.79) (width 0.3) (layer F.Cu) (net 8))
 (segment (start 113.03 102.87) (end 111.73 102.87) (width 0.3) (layer F.Cu) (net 9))
 (segment (start 111.73 102.87) (end 108.9025 102.87) (width 0.3) (layer F.Cu) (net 9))
 (segment (start 118.11 102.87) (end 113.03 102.87) (width 0.3) (layer F.Cu) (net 9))
 (segment (start 88.9 108.265) (end 86.04 108.265) (width 2) (layer B.Cu) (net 13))
 (segment (start 86.04 108.265) (end 82.55 104.775) (width 2) (layer B.Cu) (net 13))
 (segment (start 88.9 113.265) (end 85.96 113.265) (width 2) (layer B.Cu) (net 14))
 (segment (start 85.96 113.265) (end 82.55 109.855) (width 2) (layer B.Cu) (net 14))
 (segment (start 82.55 89.535) (end 81.121484 89.535) (width 2) (layer B.Cu) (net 15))
 (segment (start 81.121484 89.535) (end 78.74 91.916484) (width 2) (layer B.Cu) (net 15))
 (segment (start 80.74168 99.695) (end 82.55 99.695) (width 2) (layer B.Cu) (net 15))
 (segment (start 78.74 91.916484) (end 78.74 97.69332) (width 2) (layer B.Cu) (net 15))
 (segment (start 78.74 97.69332) (end 80.74168 99.695) (width 2) (layer B.Cu) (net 15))
 (segment (start 105.5 83.342) (end 107.949377 85.791377) (width 0.3) (layer F.Cu) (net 6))
 (segment (start 107.949377 85.791377) (end 107.949377 101.374123) (width 0.3) (layer F.Cu) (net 6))
 (segment (start 107.949377 101.374123) (end 106.9975 102.326) (width 0.3) (layer F.Cu) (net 6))
 (segment (start 106.9975 102.326) (end 106.9975 102.87) (width 0.3) (layer F.Cu) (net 6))
 (segment (start 106.9975 102.87) (end 104.68102 102.87) (width 0.3) (layer F.Cu) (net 6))
 (segment (start 106.77398 105.41) (end 106.77398 103.09352) (width 0.3) (layer F.Cu) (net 6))
 (segment (start 106.77398 103.09352) (end 106.9975 102.87) (width 0.3) (layer F.Cu) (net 6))
 (segment (start 94.615 106.36) (end 93.115001 104.860001) (width 2) (layer B.Cu) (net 12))
 (segment (start 93.115001 104.860001) (end 90.495001 104.860001) (width 2) (layer B.Cu) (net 12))
 (segment (start 90.495001 104.860001) (end 90.399999 104.764999) (width 2) (layer B.Cu) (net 12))
 (segment (start 90.399999 104.764999) (end 88.9 103.265) (width 2) (layer B.Cu) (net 12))
 (segment (start 94.615 101.36) (end 92.310016 99.055016) (width 2) (layer B.Cu) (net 16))
 (segment (start 92.310016 99.055016) (end 86.990016 99.055016) (width 2) (layer B.Cu) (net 16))
 (segment (start 86.990016 99.055016) (end 83.549999 95.614999) (width 2) (layer B.Cu) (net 16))
 (segment (start 83.549999 95.614999) (end 82.55 94.615) (width 2) (layer B.Cu) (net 16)))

